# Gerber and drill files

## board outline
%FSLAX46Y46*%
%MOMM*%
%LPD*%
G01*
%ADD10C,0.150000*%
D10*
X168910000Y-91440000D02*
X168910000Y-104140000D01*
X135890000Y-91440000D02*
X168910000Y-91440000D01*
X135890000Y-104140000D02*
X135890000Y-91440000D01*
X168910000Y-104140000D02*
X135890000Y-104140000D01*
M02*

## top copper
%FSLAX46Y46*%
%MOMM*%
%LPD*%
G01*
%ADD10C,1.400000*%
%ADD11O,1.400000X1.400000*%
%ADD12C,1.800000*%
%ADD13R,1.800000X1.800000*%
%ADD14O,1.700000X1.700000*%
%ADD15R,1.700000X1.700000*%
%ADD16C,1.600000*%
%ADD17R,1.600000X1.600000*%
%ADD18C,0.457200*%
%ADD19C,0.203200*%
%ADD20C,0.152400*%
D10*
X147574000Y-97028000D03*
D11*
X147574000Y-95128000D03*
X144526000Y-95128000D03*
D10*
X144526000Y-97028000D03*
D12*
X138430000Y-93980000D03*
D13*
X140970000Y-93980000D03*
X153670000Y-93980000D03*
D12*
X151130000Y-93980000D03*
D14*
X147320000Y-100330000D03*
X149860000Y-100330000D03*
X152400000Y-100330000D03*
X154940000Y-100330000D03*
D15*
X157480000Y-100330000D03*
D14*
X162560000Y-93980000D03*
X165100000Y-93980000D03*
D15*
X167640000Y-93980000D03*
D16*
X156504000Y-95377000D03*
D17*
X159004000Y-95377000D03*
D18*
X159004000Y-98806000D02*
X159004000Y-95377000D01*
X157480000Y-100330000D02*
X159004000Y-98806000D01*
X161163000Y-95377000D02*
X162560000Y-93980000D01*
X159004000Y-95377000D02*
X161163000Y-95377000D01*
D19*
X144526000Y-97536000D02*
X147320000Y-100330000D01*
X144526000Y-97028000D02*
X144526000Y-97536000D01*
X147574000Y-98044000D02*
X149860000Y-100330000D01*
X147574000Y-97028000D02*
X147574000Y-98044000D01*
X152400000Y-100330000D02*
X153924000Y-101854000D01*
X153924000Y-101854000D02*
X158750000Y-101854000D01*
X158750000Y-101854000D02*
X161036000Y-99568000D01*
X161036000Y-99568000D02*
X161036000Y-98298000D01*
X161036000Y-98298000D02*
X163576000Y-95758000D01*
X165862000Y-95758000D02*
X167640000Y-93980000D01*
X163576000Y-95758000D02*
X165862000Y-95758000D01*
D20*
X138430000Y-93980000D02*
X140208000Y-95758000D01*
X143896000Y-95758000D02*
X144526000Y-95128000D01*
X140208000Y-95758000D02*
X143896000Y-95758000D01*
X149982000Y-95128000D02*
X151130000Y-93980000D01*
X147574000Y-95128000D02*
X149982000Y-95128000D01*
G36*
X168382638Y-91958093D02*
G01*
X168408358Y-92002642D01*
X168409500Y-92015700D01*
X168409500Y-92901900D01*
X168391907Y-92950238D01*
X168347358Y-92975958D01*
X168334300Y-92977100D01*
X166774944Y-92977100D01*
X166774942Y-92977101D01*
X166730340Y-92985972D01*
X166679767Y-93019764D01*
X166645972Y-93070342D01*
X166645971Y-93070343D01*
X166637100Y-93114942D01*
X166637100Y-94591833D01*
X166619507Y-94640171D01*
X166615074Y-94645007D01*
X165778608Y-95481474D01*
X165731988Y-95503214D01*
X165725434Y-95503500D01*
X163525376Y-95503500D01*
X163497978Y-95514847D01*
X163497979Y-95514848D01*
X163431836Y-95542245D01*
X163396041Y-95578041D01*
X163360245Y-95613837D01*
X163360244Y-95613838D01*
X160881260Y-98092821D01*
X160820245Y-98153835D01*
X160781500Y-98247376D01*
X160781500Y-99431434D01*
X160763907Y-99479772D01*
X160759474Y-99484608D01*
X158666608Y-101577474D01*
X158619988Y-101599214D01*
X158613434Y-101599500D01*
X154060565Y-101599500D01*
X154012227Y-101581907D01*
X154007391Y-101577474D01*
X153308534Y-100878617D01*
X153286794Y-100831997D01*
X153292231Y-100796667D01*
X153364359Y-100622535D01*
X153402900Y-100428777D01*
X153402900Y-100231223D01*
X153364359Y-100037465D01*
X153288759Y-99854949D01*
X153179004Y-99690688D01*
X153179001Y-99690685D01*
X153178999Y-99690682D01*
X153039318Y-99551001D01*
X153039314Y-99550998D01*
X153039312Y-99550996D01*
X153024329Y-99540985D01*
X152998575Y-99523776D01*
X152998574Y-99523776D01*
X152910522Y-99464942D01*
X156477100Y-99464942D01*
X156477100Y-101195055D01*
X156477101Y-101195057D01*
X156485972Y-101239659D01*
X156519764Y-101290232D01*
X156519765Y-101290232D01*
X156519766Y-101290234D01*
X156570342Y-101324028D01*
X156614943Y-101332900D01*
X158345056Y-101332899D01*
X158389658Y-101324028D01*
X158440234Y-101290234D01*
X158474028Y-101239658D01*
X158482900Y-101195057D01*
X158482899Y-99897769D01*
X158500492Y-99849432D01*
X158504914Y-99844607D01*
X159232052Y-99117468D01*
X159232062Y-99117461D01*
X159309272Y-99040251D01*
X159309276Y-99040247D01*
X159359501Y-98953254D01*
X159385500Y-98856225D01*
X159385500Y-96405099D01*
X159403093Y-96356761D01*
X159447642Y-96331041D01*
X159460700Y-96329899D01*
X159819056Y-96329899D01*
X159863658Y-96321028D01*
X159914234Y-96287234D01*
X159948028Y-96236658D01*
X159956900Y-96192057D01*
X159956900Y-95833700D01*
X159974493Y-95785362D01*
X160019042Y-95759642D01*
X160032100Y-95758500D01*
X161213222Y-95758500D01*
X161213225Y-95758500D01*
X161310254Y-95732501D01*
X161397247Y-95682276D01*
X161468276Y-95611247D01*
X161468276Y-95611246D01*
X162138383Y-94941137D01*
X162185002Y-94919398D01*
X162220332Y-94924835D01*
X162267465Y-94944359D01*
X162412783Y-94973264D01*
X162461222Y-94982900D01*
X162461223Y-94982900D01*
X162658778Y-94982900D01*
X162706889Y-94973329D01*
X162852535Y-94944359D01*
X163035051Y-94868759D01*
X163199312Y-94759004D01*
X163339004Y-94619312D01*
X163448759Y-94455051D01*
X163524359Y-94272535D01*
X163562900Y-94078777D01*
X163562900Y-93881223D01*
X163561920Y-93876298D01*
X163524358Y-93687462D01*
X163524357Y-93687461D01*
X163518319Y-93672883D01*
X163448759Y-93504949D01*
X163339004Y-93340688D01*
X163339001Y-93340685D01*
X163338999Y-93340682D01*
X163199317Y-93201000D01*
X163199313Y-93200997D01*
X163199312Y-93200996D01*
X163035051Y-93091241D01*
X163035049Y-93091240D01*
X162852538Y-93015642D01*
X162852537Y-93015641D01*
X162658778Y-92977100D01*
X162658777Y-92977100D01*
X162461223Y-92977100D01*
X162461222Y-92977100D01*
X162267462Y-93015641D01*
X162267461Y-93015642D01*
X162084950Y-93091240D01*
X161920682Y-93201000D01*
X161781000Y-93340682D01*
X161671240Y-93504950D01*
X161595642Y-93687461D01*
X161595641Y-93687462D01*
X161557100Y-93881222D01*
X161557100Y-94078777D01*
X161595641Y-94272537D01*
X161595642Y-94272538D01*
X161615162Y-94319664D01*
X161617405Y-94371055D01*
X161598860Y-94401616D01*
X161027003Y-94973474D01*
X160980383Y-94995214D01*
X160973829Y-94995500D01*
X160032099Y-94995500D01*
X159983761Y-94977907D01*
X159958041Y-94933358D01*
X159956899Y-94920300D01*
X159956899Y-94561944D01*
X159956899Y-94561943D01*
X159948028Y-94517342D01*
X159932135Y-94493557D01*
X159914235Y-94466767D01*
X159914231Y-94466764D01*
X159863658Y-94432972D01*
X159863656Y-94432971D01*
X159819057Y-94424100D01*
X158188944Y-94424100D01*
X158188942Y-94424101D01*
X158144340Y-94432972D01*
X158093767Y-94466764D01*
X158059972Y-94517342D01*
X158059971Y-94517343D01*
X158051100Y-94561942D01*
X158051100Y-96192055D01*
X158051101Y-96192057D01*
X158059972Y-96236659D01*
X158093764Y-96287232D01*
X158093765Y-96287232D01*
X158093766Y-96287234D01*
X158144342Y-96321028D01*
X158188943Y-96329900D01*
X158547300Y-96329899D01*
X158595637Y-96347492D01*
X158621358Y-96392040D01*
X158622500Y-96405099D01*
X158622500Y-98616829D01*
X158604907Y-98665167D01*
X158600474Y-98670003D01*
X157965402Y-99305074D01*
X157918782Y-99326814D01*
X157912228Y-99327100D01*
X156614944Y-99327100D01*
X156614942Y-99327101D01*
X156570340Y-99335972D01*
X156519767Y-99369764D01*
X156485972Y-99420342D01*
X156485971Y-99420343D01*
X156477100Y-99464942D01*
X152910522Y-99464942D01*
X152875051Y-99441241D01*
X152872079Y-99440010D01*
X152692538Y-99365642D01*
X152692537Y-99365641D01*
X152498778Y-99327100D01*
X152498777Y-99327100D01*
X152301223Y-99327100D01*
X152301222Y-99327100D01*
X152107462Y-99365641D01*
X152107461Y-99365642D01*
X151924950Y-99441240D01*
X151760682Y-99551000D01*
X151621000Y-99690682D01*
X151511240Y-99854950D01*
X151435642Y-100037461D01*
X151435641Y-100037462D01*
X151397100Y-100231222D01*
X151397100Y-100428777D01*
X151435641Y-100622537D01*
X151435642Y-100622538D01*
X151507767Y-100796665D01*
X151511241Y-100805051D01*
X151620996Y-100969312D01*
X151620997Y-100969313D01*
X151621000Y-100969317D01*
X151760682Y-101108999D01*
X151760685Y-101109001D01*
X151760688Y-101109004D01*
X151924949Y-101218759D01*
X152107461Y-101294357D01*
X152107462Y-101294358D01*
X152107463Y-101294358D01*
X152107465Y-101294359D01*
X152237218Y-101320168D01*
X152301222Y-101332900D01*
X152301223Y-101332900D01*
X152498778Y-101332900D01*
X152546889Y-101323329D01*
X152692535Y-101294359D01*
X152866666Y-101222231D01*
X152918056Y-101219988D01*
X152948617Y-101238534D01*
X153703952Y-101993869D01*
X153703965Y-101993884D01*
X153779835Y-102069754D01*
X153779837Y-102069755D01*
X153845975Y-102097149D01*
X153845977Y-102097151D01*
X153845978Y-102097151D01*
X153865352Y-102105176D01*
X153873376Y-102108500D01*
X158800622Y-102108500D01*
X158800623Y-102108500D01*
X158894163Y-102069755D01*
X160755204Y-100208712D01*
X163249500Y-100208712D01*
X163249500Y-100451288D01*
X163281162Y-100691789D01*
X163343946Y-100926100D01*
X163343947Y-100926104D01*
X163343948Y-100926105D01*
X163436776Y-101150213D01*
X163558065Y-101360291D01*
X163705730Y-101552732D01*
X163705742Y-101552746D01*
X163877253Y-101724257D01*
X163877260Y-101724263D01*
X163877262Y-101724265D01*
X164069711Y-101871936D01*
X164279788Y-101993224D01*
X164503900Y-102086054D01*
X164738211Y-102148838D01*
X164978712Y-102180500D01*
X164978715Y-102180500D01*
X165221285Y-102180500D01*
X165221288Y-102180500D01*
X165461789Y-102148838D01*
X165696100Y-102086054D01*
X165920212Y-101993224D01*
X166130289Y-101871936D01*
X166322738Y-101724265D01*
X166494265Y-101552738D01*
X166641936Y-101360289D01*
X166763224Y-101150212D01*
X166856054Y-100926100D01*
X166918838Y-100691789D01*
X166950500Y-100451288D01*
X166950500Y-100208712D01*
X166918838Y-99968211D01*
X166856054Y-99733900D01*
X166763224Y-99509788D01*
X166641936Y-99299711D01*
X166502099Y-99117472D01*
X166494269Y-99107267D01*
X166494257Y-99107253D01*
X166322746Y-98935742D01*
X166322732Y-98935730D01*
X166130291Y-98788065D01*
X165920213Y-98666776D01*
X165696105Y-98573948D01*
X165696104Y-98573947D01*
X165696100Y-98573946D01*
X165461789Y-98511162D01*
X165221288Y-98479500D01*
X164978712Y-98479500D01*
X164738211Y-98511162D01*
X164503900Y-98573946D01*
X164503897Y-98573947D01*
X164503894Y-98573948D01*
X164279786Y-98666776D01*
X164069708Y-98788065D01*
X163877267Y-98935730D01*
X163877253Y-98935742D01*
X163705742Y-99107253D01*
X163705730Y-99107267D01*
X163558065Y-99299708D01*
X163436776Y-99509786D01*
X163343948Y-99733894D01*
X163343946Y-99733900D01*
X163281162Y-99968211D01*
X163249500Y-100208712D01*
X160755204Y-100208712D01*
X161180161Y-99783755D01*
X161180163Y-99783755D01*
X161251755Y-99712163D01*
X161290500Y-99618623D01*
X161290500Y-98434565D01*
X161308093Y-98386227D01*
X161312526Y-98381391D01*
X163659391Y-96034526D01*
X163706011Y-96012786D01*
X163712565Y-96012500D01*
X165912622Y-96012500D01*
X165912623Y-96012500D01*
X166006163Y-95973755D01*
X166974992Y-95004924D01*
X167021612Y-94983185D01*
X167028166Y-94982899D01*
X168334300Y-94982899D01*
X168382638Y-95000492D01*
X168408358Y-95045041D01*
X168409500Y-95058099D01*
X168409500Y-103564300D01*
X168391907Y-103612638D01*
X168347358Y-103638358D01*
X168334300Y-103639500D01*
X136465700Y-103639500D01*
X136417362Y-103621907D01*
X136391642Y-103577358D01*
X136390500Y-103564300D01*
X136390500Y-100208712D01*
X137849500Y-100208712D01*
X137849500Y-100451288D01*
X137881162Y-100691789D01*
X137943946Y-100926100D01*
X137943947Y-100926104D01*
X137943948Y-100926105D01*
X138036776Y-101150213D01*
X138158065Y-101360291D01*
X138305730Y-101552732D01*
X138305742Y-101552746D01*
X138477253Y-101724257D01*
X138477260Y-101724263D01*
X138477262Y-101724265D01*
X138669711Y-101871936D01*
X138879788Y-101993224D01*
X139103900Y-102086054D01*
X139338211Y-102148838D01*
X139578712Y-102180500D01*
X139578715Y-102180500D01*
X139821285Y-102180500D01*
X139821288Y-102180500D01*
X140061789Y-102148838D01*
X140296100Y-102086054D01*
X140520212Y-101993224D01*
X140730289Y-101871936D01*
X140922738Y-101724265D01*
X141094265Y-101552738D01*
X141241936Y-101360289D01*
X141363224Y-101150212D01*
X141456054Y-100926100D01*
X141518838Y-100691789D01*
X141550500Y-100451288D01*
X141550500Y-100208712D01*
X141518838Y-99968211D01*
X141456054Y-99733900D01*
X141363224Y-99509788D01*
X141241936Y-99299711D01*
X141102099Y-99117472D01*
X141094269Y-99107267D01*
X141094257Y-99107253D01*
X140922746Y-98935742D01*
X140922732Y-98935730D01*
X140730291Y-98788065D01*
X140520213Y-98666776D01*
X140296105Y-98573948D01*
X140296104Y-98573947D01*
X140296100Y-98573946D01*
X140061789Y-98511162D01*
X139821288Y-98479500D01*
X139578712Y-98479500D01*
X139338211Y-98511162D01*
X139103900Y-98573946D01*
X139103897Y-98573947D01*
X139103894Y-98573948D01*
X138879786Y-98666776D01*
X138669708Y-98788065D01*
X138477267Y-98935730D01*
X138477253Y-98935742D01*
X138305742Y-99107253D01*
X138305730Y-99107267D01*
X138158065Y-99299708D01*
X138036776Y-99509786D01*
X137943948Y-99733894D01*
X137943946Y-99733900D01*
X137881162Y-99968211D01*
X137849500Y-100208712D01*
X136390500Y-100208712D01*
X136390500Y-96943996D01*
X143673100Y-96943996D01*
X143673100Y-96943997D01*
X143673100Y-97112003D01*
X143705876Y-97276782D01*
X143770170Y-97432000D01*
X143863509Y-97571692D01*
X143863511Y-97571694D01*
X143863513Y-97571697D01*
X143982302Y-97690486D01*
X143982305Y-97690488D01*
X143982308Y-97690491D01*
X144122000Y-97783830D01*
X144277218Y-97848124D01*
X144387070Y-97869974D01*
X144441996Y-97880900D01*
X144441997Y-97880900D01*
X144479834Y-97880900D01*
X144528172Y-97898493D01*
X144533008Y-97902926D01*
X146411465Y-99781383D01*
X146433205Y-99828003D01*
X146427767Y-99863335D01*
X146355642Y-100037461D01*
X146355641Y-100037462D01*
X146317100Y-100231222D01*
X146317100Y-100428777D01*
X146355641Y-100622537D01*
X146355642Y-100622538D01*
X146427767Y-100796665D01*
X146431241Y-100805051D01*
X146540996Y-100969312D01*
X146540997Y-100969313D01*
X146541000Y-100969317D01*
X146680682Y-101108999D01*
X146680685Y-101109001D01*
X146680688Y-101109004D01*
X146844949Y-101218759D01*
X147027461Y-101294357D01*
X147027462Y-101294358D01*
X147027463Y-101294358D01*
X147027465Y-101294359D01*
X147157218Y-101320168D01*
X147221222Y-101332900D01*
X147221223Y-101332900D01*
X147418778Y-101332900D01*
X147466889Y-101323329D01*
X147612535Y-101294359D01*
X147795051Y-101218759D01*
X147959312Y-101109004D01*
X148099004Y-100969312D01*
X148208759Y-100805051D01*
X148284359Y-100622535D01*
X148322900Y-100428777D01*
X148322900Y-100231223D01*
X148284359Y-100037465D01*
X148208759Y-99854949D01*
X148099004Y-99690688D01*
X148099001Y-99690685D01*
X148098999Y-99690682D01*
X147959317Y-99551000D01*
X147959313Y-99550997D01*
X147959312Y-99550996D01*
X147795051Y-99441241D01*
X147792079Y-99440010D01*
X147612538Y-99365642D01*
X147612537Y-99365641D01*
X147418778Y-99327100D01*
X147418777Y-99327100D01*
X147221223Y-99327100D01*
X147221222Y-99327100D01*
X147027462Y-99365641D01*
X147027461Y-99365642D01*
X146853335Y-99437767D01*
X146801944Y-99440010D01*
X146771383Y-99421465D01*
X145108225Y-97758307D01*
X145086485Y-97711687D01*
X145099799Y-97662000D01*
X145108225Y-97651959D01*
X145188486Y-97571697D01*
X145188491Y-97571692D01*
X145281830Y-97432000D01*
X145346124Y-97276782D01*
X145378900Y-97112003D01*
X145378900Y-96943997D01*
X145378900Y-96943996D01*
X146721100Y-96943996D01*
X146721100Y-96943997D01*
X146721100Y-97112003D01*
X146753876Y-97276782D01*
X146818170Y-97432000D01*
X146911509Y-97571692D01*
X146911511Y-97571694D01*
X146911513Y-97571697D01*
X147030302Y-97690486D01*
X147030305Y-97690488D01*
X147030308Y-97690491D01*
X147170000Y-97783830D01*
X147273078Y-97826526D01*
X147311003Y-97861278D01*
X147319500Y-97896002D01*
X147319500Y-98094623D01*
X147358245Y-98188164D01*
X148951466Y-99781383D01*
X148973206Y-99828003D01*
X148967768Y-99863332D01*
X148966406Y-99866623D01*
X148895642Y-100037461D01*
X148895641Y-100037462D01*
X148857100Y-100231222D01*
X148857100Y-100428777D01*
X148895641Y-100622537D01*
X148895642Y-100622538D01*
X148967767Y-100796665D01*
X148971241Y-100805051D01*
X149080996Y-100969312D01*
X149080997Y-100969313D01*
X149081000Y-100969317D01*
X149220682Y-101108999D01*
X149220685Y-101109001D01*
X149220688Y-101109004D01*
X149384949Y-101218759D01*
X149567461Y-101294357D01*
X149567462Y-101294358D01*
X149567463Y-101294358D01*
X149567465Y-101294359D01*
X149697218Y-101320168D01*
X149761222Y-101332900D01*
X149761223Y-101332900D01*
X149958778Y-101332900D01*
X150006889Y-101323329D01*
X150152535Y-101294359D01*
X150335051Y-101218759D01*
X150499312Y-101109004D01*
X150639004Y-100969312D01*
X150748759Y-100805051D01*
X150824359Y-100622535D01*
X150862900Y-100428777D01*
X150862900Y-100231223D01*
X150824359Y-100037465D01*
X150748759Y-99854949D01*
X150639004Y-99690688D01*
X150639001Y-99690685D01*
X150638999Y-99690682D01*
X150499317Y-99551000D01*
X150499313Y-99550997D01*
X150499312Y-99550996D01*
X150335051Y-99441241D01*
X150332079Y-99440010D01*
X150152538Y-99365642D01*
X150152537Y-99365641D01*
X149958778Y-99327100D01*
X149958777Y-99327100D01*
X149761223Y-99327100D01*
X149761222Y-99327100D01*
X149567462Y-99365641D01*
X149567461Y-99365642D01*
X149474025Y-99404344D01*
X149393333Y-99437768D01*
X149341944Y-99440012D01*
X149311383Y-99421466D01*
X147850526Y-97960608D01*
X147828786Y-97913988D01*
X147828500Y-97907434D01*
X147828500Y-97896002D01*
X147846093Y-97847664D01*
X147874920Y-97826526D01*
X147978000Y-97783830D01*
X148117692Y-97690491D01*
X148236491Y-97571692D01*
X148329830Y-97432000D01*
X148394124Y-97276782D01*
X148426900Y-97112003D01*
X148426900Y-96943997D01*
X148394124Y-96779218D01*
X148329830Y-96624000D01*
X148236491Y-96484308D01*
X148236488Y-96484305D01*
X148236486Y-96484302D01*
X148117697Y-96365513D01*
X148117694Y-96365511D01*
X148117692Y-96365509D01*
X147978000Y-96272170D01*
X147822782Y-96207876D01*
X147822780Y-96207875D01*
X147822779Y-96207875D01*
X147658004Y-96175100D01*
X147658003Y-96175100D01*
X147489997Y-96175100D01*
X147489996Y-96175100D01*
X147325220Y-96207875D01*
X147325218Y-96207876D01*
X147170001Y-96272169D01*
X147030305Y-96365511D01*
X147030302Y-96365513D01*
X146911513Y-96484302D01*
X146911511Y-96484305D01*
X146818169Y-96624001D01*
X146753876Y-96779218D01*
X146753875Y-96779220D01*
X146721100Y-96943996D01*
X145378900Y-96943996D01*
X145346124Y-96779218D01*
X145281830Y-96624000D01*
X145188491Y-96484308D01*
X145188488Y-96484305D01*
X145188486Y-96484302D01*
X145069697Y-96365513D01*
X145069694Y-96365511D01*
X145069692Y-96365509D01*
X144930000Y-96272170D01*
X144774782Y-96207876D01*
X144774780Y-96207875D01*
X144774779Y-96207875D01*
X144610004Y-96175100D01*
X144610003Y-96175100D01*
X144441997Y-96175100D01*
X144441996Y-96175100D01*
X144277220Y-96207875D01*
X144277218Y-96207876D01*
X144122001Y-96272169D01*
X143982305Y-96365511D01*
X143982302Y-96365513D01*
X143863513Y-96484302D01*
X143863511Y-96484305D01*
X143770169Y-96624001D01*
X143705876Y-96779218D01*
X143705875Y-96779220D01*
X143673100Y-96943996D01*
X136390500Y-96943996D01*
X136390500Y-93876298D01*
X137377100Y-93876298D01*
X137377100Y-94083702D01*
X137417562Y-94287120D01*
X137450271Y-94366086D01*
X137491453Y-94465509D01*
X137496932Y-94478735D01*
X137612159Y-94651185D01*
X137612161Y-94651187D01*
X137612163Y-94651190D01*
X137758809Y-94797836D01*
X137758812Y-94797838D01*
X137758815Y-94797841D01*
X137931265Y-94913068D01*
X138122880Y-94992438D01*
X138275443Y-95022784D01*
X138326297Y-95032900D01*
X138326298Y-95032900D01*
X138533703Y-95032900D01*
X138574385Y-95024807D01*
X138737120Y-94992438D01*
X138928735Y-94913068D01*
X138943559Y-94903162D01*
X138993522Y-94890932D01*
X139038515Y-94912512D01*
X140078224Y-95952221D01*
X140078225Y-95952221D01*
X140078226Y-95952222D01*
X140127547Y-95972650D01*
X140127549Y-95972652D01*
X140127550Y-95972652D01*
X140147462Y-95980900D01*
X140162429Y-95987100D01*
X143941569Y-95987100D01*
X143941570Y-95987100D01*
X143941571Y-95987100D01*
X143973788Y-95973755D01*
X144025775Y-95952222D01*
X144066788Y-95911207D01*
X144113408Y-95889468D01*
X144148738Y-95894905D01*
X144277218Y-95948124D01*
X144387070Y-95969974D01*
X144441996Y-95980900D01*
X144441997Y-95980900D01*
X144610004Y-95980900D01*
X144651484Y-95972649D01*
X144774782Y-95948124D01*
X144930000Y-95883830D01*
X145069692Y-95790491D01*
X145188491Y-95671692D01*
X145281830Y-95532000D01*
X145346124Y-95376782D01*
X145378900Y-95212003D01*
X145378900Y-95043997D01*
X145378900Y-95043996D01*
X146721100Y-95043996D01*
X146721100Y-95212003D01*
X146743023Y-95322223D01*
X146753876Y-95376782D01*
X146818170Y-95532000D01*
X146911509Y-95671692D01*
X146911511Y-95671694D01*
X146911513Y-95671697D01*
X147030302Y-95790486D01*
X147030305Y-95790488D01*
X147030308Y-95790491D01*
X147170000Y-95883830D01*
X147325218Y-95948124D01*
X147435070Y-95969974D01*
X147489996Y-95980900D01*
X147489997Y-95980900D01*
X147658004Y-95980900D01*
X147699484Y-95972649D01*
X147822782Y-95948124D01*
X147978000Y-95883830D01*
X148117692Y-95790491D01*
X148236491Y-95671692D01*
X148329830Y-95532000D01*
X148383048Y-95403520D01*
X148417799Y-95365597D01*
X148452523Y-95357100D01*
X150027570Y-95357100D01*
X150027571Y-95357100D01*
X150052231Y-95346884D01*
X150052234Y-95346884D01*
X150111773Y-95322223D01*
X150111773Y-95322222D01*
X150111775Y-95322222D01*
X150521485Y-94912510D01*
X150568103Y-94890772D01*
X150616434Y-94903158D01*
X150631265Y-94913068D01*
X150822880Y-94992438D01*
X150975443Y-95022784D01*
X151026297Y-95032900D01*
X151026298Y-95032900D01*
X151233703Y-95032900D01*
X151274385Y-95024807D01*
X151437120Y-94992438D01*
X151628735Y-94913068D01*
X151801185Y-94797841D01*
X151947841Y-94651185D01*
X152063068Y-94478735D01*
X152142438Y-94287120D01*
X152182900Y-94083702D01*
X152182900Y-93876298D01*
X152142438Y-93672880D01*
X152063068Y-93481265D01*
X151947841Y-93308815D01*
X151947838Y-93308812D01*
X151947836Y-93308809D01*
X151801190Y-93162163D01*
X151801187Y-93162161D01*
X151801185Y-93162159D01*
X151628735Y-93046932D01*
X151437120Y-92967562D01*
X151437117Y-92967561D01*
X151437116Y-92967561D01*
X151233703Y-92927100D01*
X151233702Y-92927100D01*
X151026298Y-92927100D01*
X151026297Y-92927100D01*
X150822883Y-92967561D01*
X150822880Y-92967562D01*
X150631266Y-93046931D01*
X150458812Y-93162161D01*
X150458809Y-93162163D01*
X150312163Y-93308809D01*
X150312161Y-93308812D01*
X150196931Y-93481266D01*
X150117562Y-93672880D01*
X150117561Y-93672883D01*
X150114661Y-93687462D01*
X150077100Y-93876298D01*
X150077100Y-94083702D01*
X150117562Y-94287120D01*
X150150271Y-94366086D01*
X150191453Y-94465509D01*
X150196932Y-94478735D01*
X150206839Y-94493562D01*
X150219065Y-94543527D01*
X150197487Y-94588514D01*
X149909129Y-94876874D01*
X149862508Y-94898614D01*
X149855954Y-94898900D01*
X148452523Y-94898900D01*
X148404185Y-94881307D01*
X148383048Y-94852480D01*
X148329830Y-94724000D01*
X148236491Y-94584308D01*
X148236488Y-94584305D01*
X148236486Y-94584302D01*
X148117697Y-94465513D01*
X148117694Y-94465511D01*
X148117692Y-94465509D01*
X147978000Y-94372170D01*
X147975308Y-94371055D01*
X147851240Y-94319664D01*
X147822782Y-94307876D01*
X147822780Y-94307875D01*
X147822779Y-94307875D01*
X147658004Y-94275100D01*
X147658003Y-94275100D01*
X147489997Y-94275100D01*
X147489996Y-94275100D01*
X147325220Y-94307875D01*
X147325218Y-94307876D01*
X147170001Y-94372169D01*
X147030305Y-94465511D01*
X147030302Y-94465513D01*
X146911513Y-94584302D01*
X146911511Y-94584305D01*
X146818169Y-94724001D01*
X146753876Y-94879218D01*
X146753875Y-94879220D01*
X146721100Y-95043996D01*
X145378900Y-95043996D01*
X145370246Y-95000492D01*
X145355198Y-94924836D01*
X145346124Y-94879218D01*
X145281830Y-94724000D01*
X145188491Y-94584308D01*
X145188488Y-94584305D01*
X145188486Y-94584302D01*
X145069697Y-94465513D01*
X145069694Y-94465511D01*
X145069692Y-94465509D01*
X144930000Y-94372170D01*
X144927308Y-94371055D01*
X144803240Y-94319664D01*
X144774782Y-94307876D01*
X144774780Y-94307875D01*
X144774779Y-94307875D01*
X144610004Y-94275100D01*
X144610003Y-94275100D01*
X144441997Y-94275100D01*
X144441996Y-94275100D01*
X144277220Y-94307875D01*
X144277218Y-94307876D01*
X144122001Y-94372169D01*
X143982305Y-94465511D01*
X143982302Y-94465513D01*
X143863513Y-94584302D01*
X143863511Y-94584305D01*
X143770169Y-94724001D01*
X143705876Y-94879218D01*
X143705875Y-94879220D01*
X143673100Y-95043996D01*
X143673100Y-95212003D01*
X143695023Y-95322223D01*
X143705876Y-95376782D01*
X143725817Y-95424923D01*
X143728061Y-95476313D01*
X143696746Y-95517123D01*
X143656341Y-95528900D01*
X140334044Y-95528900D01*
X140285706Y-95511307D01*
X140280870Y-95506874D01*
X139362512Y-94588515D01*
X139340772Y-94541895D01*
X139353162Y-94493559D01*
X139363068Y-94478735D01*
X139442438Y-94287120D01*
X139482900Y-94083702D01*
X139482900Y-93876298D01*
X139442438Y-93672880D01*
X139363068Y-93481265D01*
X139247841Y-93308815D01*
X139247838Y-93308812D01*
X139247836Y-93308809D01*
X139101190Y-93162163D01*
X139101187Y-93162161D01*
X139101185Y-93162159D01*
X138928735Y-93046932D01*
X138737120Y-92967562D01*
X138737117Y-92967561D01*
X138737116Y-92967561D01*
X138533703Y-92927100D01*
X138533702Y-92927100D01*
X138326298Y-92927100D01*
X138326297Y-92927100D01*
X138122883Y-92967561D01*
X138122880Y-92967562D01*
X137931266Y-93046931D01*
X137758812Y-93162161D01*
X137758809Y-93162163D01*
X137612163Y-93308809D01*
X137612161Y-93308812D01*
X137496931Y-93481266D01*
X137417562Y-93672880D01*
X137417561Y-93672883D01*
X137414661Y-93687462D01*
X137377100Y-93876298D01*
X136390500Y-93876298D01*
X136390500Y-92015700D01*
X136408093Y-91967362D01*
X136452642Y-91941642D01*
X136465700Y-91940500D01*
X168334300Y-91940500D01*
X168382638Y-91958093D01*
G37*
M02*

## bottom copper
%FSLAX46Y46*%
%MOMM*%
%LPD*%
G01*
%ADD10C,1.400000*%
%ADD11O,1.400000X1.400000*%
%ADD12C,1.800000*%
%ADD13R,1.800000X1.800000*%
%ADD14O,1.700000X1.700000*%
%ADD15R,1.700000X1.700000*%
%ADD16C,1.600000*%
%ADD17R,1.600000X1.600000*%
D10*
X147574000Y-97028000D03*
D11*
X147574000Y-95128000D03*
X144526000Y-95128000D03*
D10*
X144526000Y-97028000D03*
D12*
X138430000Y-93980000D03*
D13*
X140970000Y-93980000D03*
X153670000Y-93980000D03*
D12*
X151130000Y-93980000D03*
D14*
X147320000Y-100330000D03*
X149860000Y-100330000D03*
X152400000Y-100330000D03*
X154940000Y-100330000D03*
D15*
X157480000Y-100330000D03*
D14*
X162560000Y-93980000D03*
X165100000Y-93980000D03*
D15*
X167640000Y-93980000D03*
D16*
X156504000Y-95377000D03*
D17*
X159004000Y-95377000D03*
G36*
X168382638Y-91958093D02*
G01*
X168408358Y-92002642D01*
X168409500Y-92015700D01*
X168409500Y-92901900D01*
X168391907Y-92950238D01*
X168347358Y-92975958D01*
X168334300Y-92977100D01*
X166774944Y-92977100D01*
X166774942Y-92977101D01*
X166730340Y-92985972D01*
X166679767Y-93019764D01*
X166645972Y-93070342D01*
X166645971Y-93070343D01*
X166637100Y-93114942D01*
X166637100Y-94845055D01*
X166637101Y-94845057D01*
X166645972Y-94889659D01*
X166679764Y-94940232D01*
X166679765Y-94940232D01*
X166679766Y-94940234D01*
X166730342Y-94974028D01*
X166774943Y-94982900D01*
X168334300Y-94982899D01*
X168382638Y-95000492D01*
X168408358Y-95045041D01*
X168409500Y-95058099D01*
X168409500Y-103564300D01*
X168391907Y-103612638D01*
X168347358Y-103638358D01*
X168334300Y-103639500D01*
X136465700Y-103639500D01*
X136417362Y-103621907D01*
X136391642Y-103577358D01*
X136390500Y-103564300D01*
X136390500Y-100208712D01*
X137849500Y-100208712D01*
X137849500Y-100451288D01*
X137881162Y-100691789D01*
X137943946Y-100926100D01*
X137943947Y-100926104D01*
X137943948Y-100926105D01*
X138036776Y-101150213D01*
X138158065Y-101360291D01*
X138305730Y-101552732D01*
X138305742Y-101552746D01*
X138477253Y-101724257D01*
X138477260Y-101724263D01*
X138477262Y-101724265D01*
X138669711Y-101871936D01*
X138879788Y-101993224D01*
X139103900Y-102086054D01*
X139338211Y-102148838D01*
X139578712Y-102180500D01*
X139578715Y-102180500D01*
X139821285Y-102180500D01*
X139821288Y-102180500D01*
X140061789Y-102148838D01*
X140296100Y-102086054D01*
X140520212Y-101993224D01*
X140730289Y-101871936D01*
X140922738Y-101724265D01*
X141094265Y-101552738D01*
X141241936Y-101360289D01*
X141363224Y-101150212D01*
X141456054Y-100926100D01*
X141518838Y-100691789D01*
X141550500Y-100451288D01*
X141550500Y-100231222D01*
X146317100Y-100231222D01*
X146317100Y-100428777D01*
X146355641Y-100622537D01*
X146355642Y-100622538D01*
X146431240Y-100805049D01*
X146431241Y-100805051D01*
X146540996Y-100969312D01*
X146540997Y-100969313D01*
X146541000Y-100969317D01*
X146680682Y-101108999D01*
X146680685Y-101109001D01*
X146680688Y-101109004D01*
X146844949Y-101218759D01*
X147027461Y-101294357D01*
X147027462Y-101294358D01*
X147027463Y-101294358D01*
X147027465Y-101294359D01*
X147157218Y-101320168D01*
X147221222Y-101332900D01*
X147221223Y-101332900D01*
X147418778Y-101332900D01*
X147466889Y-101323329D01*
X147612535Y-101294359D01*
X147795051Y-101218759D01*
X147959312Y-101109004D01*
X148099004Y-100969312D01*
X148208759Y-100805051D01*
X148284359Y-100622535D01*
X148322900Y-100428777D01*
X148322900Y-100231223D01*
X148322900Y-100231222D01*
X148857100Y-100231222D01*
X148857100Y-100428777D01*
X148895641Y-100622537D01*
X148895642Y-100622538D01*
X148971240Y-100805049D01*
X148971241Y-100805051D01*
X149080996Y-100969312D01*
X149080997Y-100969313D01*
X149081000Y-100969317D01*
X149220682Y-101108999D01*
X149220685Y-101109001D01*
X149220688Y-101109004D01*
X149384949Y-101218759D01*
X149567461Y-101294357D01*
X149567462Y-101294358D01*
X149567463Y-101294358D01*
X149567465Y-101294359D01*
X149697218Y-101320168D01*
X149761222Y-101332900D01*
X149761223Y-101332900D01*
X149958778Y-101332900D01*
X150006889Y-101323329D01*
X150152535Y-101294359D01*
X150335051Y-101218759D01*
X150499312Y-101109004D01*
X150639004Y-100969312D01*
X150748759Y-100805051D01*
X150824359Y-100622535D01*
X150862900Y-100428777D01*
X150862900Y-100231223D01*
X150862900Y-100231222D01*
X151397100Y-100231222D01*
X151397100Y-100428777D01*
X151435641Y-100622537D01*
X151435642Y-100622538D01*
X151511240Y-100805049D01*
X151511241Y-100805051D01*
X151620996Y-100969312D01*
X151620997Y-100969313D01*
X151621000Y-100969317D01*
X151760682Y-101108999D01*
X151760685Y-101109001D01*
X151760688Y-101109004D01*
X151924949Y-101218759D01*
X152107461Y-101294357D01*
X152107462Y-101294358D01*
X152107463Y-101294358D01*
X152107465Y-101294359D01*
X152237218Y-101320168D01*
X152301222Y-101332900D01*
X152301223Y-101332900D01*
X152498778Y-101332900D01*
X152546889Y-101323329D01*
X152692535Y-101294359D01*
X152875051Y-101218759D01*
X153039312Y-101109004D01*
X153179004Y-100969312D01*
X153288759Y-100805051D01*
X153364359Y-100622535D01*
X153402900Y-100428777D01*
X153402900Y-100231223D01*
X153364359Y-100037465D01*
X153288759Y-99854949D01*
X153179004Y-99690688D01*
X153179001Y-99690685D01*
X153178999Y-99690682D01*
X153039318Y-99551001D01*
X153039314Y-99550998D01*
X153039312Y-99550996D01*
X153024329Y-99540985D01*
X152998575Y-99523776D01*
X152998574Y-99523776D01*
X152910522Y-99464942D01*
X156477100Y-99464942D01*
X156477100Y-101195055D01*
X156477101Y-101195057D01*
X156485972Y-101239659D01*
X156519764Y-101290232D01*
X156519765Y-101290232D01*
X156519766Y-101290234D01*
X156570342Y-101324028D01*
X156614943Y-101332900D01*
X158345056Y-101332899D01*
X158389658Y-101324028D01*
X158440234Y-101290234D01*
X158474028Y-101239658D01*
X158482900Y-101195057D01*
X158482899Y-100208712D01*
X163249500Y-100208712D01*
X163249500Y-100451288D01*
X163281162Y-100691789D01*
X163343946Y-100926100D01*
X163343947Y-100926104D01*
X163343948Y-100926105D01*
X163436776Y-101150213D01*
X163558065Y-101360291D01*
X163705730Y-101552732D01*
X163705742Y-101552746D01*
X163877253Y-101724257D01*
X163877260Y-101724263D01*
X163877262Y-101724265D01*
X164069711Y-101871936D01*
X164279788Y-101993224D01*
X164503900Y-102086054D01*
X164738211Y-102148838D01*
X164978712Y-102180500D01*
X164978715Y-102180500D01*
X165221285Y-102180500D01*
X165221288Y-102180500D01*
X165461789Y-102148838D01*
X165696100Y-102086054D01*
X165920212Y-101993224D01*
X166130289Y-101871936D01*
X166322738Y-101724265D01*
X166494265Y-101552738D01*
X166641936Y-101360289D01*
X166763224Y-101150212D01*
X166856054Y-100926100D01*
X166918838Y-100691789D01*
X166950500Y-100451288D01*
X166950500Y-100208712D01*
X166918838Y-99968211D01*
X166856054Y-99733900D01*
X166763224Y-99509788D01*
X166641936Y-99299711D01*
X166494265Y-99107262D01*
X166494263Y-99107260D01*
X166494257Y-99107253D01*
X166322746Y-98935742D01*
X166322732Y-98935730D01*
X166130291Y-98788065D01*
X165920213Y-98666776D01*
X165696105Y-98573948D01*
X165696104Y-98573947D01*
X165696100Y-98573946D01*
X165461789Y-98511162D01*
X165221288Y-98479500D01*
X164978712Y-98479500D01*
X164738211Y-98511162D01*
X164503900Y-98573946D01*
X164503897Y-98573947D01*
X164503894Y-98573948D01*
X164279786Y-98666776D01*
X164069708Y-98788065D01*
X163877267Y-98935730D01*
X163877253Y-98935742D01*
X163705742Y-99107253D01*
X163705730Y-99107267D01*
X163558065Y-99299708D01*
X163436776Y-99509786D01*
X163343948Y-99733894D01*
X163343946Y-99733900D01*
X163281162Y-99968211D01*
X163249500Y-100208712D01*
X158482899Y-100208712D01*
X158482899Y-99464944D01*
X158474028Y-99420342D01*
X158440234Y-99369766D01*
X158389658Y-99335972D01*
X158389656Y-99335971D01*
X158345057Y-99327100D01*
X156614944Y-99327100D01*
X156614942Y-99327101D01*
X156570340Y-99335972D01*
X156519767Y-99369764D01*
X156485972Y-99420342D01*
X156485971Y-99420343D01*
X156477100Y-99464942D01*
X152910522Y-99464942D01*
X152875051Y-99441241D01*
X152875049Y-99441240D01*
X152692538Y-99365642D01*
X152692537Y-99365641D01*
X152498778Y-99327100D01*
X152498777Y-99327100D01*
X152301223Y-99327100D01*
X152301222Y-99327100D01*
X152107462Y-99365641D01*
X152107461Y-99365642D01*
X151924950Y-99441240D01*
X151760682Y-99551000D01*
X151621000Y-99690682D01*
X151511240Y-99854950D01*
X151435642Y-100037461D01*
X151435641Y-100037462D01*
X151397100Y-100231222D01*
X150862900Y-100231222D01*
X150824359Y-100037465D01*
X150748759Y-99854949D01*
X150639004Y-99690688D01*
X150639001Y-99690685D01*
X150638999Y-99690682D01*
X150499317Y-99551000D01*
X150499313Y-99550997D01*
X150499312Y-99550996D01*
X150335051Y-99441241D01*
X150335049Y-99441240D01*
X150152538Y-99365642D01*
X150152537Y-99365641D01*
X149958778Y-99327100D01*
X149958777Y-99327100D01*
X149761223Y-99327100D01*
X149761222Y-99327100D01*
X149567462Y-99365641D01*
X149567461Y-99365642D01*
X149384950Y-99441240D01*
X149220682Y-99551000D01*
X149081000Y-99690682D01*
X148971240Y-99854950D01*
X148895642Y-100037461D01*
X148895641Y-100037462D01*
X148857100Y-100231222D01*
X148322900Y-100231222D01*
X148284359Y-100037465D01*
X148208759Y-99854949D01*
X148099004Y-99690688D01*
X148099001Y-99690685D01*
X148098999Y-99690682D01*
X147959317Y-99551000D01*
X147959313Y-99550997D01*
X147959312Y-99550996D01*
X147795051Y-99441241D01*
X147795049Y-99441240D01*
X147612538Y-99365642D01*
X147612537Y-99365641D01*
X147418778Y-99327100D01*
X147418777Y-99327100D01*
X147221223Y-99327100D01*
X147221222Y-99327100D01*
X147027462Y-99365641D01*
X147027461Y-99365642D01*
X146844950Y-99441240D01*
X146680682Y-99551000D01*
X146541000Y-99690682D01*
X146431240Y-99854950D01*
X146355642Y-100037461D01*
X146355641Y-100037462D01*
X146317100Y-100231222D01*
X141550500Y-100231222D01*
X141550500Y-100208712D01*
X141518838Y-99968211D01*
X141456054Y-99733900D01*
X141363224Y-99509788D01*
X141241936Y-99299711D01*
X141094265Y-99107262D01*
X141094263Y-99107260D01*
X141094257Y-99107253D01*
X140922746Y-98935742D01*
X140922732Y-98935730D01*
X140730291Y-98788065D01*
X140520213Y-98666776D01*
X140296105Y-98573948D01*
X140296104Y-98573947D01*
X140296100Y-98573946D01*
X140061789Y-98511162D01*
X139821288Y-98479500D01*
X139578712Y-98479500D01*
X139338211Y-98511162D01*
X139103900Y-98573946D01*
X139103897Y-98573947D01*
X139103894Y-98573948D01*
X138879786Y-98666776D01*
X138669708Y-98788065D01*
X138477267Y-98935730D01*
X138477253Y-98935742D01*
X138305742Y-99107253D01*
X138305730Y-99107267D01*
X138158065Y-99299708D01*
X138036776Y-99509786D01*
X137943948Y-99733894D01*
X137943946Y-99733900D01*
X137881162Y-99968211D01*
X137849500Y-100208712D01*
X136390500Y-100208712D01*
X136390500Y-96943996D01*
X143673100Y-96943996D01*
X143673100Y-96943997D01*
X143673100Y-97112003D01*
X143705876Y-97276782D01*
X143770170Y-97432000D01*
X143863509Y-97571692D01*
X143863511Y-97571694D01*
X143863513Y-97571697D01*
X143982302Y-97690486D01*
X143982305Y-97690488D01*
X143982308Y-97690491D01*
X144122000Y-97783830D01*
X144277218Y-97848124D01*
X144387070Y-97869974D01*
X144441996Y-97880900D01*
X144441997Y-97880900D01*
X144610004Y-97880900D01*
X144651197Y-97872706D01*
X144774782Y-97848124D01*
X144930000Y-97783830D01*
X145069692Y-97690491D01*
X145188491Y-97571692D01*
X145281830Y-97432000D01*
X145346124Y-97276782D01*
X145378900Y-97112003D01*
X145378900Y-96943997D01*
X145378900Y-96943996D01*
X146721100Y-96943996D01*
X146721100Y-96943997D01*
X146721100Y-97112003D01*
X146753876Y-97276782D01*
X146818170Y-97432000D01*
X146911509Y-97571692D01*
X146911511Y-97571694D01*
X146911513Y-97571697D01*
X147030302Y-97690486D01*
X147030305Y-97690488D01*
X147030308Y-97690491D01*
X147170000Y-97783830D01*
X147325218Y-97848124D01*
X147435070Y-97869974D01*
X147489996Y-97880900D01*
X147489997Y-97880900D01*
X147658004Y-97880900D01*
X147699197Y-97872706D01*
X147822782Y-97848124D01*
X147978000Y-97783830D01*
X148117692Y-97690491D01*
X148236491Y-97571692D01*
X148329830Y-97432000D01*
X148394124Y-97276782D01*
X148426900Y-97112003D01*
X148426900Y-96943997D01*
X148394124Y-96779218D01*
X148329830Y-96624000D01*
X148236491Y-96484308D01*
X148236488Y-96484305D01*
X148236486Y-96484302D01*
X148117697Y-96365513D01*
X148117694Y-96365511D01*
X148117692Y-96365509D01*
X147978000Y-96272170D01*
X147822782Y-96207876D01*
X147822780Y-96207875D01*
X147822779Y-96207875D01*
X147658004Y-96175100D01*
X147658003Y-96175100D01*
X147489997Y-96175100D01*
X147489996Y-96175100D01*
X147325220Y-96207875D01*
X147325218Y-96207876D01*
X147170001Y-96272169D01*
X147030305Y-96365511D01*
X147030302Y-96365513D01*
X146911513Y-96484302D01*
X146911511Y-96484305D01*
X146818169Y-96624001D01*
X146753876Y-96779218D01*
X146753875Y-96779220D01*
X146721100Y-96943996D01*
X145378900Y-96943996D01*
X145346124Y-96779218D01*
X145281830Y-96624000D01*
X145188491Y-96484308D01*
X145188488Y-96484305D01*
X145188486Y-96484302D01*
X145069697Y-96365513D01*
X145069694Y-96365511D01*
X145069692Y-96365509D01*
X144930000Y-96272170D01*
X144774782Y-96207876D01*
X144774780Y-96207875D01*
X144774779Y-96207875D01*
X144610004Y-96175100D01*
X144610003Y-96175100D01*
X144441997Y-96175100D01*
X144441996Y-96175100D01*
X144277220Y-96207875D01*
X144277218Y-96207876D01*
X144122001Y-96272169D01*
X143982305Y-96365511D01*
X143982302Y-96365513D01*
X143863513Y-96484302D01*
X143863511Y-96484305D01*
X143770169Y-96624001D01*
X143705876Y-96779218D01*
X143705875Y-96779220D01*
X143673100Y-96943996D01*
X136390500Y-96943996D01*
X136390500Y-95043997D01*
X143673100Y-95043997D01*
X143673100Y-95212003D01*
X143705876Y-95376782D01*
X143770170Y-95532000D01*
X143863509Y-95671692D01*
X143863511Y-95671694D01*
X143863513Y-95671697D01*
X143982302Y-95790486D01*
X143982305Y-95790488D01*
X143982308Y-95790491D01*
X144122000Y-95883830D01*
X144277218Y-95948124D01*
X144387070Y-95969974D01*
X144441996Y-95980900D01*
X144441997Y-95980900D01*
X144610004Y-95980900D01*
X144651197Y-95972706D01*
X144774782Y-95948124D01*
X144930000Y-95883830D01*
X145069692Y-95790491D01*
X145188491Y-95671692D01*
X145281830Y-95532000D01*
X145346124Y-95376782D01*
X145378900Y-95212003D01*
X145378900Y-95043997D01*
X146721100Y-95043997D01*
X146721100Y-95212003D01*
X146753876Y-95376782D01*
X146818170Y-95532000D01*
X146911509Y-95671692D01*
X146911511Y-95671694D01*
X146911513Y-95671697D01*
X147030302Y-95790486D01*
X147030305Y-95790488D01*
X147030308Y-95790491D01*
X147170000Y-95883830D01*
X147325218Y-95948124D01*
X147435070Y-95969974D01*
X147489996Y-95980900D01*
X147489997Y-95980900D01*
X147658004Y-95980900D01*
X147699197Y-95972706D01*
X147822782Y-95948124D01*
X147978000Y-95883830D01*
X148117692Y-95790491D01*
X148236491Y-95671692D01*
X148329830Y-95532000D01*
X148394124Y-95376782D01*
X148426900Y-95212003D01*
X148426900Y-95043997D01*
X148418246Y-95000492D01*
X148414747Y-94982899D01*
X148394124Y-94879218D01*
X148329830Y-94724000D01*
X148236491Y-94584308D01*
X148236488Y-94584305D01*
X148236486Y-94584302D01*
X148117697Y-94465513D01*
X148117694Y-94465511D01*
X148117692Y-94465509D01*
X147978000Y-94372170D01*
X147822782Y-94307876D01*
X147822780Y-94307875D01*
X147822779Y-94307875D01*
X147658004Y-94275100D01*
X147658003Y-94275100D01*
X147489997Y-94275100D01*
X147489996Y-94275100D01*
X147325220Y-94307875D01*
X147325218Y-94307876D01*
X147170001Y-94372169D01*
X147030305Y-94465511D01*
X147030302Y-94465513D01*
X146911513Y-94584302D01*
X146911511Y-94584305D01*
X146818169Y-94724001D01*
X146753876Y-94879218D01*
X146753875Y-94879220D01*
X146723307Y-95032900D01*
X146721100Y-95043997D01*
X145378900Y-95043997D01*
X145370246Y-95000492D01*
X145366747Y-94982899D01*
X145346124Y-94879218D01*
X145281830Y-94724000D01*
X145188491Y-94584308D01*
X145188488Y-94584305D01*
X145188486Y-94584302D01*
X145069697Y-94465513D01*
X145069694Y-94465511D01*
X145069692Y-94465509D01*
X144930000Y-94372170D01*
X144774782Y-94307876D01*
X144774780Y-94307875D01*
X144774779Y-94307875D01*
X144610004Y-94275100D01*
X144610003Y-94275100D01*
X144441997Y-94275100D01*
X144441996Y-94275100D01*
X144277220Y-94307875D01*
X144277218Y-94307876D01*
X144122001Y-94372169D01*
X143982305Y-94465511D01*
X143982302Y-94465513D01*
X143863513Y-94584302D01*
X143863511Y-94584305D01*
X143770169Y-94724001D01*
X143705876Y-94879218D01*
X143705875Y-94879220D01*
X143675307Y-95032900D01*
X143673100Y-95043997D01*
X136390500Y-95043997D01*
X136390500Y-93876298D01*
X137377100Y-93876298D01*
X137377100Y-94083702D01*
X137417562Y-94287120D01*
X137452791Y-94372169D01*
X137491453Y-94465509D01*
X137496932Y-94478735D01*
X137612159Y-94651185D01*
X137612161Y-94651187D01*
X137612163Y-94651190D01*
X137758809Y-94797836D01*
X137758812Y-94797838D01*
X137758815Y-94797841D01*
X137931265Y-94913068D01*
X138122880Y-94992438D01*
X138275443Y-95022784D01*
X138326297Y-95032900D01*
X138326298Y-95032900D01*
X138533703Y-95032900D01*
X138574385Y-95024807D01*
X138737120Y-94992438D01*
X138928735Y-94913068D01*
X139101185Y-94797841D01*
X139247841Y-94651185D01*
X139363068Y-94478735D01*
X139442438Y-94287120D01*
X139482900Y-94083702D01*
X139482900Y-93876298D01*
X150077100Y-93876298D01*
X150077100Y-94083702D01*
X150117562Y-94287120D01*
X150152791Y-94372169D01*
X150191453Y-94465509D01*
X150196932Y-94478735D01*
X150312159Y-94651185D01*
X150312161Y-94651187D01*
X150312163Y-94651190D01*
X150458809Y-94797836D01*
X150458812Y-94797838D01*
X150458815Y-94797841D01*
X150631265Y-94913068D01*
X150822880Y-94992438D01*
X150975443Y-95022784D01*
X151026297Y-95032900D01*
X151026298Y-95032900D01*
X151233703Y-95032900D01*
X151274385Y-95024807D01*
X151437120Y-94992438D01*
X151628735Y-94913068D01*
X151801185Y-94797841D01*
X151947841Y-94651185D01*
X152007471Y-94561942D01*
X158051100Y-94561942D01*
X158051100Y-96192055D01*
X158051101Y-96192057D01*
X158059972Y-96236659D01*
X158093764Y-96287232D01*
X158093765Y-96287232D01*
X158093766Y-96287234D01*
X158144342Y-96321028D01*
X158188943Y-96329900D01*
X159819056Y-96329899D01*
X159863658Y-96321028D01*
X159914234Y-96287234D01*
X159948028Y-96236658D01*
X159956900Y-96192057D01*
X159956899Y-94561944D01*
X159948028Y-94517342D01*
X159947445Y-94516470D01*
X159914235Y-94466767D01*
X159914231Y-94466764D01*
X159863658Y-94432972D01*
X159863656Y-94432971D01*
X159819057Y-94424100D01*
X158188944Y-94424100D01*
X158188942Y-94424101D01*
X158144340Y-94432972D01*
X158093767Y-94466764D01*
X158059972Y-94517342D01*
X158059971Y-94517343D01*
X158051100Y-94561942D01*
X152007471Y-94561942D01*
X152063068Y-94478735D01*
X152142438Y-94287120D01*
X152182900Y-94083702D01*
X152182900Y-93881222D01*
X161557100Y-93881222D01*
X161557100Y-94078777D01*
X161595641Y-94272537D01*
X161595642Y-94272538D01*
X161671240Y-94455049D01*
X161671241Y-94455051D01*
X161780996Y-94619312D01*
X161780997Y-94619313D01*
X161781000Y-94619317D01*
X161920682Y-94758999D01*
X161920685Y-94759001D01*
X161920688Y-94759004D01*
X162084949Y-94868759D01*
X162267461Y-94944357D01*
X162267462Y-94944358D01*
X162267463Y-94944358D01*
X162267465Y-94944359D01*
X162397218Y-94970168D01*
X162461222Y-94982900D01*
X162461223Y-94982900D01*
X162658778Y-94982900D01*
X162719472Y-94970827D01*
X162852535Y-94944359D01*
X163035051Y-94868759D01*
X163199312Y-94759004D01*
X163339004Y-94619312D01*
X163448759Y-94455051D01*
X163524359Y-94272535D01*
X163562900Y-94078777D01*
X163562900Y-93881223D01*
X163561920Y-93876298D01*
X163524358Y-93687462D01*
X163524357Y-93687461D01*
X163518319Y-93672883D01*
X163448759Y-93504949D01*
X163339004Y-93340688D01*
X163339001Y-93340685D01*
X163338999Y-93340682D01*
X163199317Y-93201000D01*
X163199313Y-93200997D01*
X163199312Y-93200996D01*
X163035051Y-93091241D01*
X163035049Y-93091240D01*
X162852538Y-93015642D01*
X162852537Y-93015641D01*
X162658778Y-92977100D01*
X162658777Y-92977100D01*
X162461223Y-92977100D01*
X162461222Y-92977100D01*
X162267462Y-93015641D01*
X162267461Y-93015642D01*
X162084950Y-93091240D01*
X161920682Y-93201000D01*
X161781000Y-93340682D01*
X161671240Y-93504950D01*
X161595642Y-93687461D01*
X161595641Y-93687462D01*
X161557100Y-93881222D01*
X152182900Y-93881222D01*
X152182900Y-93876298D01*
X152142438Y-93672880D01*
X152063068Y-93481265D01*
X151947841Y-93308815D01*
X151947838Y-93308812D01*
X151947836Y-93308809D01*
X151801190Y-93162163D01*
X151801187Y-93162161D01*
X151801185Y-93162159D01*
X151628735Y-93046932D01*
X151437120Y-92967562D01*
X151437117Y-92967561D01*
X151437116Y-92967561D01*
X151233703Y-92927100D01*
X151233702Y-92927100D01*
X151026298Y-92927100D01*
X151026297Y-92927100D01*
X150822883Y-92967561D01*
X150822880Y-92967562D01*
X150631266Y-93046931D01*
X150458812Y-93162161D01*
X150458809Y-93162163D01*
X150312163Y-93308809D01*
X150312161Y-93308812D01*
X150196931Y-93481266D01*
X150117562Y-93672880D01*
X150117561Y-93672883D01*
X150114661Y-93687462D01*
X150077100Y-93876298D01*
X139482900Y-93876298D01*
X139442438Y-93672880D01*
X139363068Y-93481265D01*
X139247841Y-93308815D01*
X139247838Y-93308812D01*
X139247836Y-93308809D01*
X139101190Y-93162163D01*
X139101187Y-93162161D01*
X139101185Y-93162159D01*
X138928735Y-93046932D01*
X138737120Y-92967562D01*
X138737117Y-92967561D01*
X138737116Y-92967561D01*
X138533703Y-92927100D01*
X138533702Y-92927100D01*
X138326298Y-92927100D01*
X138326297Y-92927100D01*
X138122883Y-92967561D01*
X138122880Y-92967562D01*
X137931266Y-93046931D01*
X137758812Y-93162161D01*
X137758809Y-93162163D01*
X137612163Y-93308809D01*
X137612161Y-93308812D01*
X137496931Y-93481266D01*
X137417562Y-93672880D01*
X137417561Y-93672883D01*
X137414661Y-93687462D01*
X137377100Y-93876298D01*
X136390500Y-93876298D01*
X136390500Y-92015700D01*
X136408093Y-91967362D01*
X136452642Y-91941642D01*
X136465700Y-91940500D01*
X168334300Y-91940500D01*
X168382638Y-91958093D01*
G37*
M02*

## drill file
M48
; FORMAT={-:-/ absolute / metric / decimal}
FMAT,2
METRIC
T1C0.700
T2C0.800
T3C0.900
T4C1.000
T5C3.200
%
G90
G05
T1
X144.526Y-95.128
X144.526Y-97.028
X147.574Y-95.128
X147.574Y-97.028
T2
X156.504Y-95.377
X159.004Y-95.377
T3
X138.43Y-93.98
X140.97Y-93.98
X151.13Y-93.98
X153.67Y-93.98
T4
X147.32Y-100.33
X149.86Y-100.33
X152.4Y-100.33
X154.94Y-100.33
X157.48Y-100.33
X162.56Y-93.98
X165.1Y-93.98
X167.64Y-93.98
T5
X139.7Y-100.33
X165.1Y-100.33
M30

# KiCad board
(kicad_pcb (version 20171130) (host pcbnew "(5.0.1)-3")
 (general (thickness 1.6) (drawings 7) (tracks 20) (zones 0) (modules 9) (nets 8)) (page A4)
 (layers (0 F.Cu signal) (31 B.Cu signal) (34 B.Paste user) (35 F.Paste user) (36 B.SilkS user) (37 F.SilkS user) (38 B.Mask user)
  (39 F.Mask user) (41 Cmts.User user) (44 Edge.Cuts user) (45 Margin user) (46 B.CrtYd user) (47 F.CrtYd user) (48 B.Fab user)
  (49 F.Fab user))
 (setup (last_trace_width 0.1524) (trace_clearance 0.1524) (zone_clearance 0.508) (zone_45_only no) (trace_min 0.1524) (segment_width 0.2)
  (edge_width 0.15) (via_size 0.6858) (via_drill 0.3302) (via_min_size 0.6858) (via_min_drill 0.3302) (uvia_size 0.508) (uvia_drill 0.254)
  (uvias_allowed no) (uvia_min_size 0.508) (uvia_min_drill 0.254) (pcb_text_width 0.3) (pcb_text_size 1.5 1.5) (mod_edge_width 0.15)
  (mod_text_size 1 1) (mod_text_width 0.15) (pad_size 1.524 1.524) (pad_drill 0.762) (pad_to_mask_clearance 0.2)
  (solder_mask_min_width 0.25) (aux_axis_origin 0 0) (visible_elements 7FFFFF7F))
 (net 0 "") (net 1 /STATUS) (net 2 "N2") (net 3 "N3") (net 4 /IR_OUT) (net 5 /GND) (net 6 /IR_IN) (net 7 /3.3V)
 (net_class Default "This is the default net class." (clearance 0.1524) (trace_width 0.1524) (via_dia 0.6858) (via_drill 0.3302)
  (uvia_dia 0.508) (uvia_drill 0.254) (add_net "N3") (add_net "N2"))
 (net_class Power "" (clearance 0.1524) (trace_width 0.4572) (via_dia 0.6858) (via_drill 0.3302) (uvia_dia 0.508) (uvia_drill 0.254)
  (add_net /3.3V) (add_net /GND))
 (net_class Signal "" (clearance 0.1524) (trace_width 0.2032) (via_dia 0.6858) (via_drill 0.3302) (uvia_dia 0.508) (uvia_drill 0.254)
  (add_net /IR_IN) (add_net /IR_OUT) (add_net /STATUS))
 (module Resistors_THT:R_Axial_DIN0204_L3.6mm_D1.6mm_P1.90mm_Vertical (layer F.Cu) (at 147.574 97.028 90)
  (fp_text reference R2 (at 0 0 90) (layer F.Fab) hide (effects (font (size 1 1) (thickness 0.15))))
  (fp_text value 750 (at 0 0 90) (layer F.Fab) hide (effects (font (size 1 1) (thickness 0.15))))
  (pad 1 thru_hole circle (at 0 0 90) (size 1.4 1.4) (drill 0.7) (layers *.Cu *.Mask) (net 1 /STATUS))
  (pad 2 thru_hole oval (at 1.9 0 90) (size 1.4 1.4) (drill 0.7) (layers *.Cu *.Mask) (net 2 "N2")))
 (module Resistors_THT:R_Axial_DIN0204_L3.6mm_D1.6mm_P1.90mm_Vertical (layer F.Cu) (at 144.526 97.028 90)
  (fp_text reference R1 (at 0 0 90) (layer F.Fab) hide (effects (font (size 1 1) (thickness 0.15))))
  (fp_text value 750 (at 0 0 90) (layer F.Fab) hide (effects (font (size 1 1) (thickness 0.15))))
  (pad 2 thru_hole oval (at 1.9 0 90) (size 1.4 1.4) (drill 0.7) (layers *.Cu *.Mask) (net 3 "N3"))
  (pad 1 thru_hole circle (at 0 0 90) (size 1.4 1.4) (drill 0.7) (layers *.Cu *.Mask) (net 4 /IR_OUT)))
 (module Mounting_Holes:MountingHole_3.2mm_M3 (layer F.Cu) (at 165.1 100.33)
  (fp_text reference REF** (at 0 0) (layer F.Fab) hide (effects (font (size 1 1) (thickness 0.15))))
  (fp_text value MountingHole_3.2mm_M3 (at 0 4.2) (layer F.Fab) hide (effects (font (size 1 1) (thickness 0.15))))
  (pad 1 np_thru_hole circle (at 0 0) (size 3.2 3.2) (drill 3.2) (layers *.Cu *.Mask)))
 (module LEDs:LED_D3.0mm (layer F.Cu) (at 140.97 93.98 180)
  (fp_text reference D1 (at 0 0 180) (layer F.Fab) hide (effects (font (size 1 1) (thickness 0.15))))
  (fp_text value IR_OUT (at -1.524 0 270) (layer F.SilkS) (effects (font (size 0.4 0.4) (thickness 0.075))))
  (pad 2 thru_hole circle (at 2.54 0 180) (size 1.8 1.8) (drill 0.9) (layers *.Cu *.Mask) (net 3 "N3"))
  (pad 1 thru_hole rect (at 0 0 180) (size 1.8 1.8) (drill 0.9) (layers *.Cu *.Mask) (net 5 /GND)))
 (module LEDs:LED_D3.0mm (layer F.Cu) (at 153.67 93.98 180)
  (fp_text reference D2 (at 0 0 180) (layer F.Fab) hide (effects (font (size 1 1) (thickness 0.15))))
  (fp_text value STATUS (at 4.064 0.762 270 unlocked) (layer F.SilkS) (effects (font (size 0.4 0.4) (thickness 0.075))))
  (pad 1 thru_hole rect (at 0 0 180) (size 1.8 1.8) (drill 0.9) (layers *.Cu *.Mask) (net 5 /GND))
  (pad 2 thru_hole circle (at 2.54 0 180) (size 1.8 1.8) (drill 0.9) (layers *.Cu *.Mask) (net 2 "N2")))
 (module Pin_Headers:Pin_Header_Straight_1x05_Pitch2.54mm (layer F.Cu) (at 157.48 100.33 270)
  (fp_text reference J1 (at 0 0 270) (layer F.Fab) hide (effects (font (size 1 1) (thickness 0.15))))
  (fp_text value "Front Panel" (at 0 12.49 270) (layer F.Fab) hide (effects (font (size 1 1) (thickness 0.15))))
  (pad 5 thru_hole oval (at 0 10.16 270) (size 1.7 1.7) (drill 1) (layers *.Cu *.Mask) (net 4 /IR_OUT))
  (pad 4 thru_hole oval (at 0 7.62 270) (size 1.7 1.7) (drill 1) (layers *.Cu *.Mask) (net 1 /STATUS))
  (pad 3 thru_hole oval (at 0 5.08 270) (size 1.7 1.7) (drill 1) (layers *.Cu *.Mask) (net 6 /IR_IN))
  (pad 2 thru_hole oval (at 0 2.54 270) (size 1.7 1.7) (drill 1) (layers *.Cu *.Mask) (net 5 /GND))
  (pad 1 thru_hole rect (at 0 0 270) (size 1.7 1.7) (drill 1) (layers *.Cu *.Mask) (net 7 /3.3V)))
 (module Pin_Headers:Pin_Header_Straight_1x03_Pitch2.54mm (layer F.Cu) (at 167.64 93.98 270)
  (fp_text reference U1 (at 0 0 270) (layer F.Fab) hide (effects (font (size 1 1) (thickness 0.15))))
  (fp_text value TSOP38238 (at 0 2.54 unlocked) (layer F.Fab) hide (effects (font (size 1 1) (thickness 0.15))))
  (pad 3 thru_hole oval (at 0 5.08 270) (size 1.7 1.7) (drill 1) (layers *.Cu *.Mask) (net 7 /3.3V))
  (pad 2 thru_hole oval (at 0 2.54 270) (size 1.7 1.7) (drill 1) (layers *.Cu *.Mask) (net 5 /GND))
  (pad 1 thru_hole rect (at 0 0 270) (size 1.7 1.7) (drill 1) (layers *.Cu *.Mask) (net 6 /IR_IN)))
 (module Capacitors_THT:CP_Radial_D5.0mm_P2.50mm (layer F.Cu) (at 159.004 95.377 180)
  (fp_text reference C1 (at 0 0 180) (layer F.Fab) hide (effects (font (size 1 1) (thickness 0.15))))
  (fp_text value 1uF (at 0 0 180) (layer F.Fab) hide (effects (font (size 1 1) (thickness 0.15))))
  (pad 2 thru_hole circle (at 2.5 0 180) (size 1.6 1.6) (drill 0.8) (layers *.Cu *.Mask) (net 5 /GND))
  (pad 1 thru_hole rect (at 0 0 180) (size 1.6 1.6) (drill 0.8) (layers *.Cu *.Mask) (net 7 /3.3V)))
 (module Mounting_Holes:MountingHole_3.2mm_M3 (layer F.Cu) (at 139.7 100.33)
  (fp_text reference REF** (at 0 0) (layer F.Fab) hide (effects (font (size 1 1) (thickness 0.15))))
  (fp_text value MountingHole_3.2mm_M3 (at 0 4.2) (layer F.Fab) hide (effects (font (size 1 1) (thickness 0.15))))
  (pad 1 np_thru_hole circle (at 0 0) (size 3.2 3.2) (drill 3.2) (layers *.Cu *.Mask)))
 (gr_line (start 168.91 91.44) (end 168.91 104.14) (layer Edge.Cuts) (width 0.15))
 (gr_line (start 135.89 91.44) (end 168.91 91.44) (layer Edge.Cuts) (width 0.15))
 (gr_line (start 135.89 104.14) (end 135.89 91.44) (layer Edge.Cuts) (width 0.15))
 (gr_line (start 168.91 104.14) (end 135.89 104.14) (layer Edge.Cuts) (width 0.15))
 (segment (start 159.004 98.806) (end 159.004 95.377) (width 0.4572) (layer F.Cu) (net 7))
 (segment (start 157.48 100.33) (end 159.004 98.806) (width 0.4572) (layer F.Cu) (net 7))
 (segment (start 161.163 95.377) (end 162.56 93.98) (width 0.4572) (layer F.Cu) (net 7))
 (segment (start 159.004 95.377) (end 161.163 95.377) (width 0.4572) (layer F.Cu) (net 7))
 (segment (start 144.526 97.536) (end 147.32 100.33) (width 0.2032) (layer F.Cu) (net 4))
 (segment (start 144.526 97.028) (end 144.526 97.536) (width 0.2032) (layer F.Cu) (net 4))
 (segment (start 147.574 98.044) (end 149.86 100.33) (width 0.2032) (layer F.Cu) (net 1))
 (segment (start 147.574 97.028) (end 147.574 98.044) (width 0.2032) (layer F.Cu) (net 1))
 (segment (start 152.4 100.33) (end 153.924 101.854) (width 0.2032) (layer F.Cu) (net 6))
 (segment (start 153.924 101.854) (end 158.75 101.854) (width 0.2032) (layer F.Cu) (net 6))
 (segment (start 158.75 101.854) (end 161.036 99.568) (width 0.2032) (layer F.Cu) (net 6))
 (segment (start 161.036 99.568) (end 161.036 98.298) (width 0.2032) (layer F.Cu) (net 6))
 (segment (start 161.036 98.298) (end 163.576 95.758) (width 0.2032) (layer F.Cu) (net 6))
 (segment (start 165.862 95.758) (end 167.64 93.98) (width 0.2032) (layer F.Cu) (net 6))
 (segment (start 163.576 95.758) (end 165.862 95.758) (width 0.2032) (layer F.Cu) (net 6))
 (segment (start 138.43 93.98) (end 140.208 95.758) (width 0.1524) (layer F.Cu) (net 3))
 (segment (start 143.896 95.758) (end 144.526 95.128) (width 0.1524) (layer F.Cu) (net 3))
 (segment (start 140.208 95.758) (end 143.896 95.758) (width 0.1524) (layer F.Cu) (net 3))
 (segment (start 149.982 95.128) (end 151.13 93.98) (width 0.1524) (layer F.Cu) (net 2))
 (segment (start 147.574 95.128) (end 149.982 95.128) (width 0.1524) (layer F.Cu) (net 2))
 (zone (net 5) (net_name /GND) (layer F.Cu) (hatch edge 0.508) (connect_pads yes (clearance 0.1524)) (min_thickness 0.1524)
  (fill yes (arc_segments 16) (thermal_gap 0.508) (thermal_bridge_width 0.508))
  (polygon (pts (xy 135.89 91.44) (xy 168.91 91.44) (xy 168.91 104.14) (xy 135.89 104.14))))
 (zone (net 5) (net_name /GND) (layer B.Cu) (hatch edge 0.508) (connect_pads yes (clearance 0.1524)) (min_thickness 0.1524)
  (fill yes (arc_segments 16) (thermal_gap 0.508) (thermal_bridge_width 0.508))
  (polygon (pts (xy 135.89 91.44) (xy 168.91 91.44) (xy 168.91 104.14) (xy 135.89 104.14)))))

